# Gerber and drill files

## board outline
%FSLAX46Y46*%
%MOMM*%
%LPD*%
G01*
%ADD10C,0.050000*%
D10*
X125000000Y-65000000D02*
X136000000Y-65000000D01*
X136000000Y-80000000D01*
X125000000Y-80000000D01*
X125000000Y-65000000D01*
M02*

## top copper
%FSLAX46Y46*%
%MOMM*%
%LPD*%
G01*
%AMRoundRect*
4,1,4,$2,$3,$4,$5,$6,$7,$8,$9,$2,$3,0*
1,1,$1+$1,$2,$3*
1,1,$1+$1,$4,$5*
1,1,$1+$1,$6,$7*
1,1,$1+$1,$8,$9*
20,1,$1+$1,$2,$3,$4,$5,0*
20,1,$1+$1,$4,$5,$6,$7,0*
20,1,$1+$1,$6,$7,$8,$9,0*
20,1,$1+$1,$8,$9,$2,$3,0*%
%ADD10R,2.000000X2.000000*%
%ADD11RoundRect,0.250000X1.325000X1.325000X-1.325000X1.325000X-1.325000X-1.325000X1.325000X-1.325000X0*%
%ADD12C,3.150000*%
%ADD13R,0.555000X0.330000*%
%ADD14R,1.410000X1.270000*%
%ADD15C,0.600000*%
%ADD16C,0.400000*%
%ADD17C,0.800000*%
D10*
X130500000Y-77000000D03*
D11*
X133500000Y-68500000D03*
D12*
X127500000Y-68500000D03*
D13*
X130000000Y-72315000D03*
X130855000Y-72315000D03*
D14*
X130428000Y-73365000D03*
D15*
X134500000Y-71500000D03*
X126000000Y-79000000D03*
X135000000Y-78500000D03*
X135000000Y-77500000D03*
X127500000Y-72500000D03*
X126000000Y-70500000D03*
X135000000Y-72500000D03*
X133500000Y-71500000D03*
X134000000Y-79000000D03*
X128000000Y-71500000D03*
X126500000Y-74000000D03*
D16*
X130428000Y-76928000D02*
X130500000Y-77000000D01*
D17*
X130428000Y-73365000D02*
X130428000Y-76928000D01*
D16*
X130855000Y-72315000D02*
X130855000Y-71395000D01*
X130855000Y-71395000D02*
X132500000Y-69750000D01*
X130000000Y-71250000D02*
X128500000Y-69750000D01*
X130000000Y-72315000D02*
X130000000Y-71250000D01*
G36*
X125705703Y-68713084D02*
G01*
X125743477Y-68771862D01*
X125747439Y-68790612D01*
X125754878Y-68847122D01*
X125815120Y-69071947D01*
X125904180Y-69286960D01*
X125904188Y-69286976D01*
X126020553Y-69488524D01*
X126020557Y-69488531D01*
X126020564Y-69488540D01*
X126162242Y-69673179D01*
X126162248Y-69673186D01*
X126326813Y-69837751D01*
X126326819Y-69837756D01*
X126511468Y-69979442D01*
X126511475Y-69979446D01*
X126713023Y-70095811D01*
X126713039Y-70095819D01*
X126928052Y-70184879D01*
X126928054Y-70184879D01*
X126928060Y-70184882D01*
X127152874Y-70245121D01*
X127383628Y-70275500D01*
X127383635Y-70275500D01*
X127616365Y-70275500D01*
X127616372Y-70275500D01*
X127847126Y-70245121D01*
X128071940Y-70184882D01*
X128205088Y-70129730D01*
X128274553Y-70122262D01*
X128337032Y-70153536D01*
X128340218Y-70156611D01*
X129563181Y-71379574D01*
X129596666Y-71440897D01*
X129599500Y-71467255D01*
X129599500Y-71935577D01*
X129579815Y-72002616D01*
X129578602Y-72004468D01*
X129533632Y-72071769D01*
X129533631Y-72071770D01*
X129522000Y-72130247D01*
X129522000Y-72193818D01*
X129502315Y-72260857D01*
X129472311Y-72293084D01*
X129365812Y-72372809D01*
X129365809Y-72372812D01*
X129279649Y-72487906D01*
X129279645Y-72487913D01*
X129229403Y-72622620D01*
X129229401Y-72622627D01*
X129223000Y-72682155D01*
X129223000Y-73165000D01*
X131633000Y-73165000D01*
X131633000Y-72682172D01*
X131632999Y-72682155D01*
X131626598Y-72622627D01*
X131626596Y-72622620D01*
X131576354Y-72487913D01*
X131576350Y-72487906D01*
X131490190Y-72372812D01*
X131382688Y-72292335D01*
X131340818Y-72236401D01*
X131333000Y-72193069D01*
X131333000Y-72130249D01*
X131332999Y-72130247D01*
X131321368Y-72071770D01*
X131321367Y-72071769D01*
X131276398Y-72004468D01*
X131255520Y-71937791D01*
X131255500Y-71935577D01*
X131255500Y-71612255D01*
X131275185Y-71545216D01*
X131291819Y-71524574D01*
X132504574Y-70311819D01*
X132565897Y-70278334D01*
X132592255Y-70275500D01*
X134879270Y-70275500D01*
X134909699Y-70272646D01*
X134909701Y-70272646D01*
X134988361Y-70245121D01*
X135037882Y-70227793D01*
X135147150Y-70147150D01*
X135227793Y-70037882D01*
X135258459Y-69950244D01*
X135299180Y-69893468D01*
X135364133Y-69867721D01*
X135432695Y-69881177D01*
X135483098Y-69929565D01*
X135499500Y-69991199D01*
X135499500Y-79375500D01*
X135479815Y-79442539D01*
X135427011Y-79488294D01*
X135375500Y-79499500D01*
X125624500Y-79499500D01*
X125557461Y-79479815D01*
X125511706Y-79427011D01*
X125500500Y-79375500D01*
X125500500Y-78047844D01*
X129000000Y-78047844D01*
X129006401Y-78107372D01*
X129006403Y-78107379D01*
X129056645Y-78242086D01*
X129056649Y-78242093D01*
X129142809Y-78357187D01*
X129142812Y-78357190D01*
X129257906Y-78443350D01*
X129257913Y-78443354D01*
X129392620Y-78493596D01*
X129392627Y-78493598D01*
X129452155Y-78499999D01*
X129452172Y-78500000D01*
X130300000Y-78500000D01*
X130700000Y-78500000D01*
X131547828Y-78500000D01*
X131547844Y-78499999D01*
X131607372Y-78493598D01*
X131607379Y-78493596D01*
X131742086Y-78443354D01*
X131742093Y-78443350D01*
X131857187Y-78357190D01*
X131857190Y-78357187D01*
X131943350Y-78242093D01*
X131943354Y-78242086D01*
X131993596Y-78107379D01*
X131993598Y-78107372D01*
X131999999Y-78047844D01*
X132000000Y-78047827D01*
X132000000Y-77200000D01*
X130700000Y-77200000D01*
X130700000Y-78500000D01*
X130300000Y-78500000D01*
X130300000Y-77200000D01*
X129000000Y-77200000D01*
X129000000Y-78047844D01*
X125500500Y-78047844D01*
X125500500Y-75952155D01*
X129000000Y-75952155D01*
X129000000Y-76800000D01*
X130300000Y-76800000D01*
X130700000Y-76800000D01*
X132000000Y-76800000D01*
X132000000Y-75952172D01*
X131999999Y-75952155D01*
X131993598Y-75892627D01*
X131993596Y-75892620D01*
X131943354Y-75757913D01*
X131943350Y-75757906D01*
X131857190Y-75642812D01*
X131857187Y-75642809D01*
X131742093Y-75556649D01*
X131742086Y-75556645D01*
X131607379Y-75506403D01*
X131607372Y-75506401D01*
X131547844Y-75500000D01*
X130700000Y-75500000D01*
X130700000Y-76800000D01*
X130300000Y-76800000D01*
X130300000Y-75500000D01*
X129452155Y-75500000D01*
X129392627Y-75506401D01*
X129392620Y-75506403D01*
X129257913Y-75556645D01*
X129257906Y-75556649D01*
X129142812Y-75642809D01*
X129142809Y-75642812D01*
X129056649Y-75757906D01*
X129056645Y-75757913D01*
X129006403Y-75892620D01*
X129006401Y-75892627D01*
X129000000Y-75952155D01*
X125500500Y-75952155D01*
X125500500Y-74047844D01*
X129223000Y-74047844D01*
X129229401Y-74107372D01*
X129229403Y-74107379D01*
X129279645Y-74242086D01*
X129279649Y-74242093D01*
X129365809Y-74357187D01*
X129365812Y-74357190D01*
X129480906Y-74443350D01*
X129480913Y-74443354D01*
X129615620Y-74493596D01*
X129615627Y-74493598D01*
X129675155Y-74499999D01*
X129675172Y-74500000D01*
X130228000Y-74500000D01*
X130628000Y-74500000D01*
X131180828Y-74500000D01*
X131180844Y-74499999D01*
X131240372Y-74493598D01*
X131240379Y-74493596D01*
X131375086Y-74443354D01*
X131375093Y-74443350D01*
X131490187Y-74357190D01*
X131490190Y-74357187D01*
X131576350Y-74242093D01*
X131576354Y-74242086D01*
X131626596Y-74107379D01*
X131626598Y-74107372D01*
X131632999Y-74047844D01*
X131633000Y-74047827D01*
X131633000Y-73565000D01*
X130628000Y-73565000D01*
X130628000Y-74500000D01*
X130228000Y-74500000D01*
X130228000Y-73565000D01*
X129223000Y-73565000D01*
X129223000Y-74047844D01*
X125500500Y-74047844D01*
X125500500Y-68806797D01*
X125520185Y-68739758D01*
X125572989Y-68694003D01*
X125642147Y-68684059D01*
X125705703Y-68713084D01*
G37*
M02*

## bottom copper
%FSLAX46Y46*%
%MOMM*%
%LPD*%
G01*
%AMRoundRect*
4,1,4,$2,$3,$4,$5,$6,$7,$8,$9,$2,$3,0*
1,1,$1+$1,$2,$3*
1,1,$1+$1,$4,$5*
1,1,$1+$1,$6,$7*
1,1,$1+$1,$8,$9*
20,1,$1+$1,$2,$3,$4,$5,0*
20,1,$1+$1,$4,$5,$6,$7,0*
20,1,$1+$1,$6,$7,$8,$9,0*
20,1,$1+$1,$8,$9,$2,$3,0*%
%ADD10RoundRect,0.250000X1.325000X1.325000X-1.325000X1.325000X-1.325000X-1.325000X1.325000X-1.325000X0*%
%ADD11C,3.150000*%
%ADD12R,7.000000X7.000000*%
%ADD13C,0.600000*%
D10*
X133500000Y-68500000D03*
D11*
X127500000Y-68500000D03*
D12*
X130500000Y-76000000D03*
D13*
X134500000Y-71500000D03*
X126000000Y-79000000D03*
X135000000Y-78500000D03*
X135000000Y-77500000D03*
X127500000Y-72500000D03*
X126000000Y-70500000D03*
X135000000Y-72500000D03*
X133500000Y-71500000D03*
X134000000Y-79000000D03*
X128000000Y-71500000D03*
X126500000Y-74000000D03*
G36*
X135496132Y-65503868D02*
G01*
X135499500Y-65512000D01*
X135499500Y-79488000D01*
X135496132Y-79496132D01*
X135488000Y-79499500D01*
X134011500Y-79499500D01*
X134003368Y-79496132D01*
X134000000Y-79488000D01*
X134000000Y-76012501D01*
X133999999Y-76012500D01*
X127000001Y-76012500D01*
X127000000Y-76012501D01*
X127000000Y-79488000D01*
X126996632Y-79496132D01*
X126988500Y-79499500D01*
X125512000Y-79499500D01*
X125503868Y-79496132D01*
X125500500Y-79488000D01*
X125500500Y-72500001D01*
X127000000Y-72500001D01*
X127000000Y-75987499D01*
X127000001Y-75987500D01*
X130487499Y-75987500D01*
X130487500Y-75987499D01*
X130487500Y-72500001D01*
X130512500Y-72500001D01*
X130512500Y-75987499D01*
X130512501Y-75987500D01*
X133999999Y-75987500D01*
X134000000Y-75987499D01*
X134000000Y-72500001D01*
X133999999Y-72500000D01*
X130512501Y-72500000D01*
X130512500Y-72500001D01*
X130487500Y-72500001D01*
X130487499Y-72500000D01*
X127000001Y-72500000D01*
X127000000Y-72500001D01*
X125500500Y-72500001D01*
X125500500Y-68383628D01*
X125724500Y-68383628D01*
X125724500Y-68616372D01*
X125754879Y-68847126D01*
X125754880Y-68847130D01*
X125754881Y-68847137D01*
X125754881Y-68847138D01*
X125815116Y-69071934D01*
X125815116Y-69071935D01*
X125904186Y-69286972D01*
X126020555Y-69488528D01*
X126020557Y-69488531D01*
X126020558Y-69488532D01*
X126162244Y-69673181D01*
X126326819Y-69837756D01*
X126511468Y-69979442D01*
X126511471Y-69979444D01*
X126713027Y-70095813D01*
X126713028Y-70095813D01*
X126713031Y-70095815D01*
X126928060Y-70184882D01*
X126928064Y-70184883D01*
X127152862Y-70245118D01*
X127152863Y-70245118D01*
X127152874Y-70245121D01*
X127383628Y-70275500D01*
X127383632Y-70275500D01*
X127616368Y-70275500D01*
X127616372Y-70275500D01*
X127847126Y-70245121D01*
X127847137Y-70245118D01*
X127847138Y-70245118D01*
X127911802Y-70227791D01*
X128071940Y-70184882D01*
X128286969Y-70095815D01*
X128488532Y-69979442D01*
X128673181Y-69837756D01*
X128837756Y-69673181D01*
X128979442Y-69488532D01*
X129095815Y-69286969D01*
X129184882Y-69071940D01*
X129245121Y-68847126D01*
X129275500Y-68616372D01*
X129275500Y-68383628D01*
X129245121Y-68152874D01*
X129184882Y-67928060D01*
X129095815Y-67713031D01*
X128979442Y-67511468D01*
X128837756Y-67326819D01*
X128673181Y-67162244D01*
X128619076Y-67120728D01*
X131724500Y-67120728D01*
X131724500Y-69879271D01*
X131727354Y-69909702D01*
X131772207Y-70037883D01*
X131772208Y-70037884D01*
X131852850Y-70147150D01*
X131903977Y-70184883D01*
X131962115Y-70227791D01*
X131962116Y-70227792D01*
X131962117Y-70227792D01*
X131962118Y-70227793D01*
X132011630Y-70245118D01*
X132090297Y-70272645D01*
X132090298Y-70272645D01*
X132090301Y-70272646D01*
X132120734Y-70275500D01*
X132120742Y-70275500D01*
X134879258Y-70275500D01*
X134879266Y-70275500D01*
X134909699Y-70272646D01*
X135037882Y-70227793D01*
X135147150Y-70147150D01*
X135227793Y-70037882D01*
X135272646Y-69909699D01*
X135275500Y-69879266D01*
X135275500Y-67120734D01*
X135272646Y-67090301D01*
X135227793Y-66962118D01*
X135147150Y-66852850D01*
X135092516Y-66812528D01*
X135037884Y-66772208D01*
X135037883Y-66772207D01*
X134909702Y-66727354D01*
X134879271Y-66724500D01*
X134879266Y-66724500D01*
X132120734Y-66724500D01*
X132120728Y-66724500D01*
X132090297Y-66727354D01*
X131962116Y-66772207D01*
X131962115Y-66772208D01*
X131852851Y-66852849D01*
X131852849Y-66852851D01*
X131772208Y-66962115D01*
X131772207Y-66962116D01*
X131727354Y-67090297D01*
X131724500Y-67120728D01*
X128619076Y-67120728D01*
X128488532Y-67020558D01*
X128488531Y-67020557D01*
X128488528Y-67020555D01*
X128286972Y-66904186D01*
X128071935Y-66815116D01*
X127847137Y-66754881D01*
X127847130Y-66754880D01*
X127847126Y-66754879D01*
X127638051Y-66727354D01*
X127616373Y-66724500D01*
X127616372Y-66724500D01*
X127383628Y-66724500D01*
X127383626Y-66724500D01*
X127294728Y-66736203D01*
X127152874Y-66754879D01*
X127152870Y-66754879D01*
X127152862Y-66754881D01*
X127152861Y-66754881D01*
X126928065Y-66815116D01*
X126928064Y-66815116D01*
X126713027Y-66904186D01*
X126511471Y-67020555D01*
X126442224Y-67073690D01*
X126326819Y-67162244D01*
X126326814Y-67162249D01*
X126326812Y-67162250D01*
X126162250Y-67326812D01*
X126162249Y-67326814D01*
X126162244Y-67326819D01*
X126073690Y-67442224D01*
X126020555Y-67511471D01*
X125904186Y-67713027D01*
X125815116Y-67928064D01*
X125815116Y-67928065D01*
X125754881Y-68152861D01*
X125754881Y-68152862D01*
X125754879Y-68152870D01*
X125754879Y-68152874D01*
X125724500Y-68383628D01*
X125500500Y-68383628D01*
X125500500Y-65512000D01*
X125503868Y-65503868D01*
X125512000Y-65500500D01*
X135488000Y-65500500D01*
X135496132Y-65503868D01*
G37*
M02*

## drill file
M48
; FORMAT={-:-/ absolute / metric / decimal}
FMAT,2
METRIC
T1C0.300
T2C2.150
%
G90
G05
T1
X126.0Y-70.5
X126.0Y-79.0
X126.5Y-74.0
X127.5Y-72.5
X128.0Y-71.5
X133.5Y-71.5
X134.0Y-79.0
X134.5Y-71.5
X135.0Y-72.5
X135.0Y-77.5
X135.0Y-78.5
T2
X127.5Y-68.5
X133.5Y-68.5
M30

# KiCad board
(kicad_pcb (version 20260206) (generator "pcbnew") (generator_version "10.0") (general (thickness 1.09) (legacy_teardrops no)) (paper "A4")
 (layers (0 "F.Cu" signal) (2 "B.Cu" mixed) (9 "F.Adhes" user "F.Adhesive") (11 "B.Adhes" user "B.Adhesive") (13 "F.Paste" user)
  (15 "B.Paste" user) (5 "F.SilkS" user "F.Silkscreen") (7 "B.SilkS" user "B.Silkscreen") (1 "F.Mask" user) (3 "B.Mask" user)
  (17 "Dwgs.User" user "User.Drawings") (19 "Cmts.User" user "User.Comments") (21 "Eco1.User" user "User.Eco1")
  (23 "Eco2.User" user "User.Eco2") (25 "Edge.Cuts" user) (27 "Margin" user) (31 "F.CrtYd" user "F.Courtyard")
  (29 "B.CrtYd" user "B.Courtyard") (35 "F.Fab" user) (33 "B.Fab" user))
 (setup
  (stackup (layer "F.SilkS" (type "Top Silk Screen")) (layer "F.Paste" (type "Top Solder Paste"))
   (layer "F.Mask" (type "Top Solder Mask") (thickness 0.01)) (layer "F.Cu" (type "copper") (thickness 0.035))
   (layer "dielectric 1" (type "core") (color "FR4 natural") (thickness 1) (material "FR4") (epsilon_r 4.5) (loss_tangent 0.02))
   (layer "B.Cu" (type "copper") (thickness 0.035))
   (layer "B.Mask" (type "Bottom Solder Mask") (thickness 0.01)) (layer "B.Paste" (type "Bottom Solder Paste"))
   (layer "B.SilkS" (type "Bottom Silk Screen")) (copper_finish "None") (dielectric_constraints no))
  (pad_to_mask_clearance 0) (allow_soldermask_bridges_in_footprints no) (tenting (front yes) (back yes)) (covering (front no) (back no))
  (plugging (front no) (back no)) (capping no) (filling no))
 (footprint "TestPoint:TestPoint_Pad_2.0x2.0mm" (layer "F.Cu") (at 130.5 77)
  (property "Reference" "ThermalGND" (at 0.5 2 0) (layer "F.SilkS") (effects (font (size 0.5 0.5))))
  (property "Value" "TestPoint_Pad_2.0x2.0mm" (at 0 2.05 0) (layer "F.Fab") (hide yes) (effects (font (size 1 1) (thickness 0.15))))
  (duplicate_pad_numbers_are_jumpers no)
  (pad "1" smd rect (at 0 0) (size 2 2) (layers "F.Cu" "F.Mask") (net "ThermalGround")))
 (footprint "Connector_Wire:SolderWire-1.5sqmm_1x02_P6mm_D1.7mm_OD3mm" (layer "F.Cu") (at 133.5 68.5 180)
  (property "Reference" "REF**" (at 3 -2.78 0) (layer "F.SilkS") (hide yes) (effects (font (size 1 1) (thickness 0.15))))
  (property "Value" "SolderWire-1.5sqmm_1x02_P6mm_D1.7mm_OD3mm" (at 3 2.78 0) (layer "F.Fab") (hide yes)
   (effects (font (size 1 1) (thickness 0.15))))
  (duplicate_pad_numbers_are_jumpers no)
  (pad "1" thru_hole roundrect (at 0 0 180) (size 3.15 3.15) (drill 2.15) (layers "*.Cu" "*.Mask") (remove_unused_layers no)
   (roundrect_rratio 0.079365) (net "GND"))
  (pad "2" thru_hole circle (at 6 0 180) (size 3.15 3.15) (drill 2.15) (layers "*.Cu" "*.Mask") (remove_unused_layers no) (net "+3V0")))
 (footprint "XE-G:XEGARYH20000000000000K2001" (layer "F.Cu") (at 130.428 73.075)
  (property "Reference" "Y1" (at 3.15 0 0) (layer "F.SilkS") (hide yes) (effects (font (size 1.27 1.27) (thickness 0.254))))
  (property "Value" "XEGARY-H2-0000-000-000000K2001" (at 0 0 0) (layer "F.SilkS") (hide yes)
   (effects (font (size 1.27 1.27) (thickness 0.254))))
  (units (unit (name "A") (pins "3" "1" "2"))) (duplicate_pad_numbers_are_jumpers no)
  (pad "1" smd rect (at -0.428 -0.76 90) (size 0.33 0.555) (layers "F.Cu" "F.Mask" "F.Paste") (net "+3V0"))
  (pad "2" smd rect (at 0.427 -0.76 90) (size 0.33 0.555) (layers "F.Cu" "F.Mask" "F.Paste") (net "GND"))
  (pad "3" smd rect (at 0 0.29 90) (size 1.27 1.41) (layers "F.Cu" "F.Mask" "F.Paste") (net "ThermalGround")))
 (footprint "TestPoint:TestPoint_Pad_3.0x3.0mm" (layer "B.Cu") (at 130.5 76 180)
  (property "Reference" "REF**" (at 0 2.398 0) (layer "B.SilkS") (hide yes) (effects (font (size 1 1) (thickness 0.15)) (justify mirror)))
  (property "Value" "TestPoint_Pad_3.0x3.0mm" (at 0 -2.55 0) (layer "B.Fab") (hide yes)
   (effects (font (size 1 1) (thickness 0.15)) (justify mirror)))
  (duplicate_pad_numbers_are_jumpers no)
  (pad "1" smd rect (at 0 0 180) (size 7 7) (layers "B.Cu" "B.Mask") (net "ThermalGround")))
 (gr_rect (start 125 65) (end 136 80) (stroke (width 0.05) (type default)) (fill no) (layer "Edge.Cuts"))
 (segment (start 130.428 76.928) (end 130.5 77) (width 0.4) (layer "F.Cu") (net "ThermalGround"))
 (segment (start 130.428 73.365) (end 130.428 76.928) (width 0.8) (layer "F.Cu") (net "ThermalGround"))
 (via (at 134.5 71.5) (size 0.6) (drill 0.3) (layers "F.Cu" "B.Cu") (free yes) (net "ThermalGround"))
 (via (at 126 79) (size 0.6) (drill 0.3) (layers "F.Cu" "B.Cu") (free yes) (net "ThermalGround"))
 (via (at 135 78.5) (size 0.6) (drill 0.3) (layers "F.Cu" "B.Cu") (free yes) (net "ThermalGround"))
 (via (at 135 77.5) (size 0.6) (drill 0.3) (layers "F.Cu" "B.Cu") (free yes) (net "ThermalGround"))
 (via (at 127.5 72.5) (size 0.6) (drill 0.3) (layers "F.Cu" "B.Cu") (free yes) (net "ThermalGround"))
 (via (at 126 70.5) (size 0.6) (drill 0.3) (layers "F.Cu" "B.Cu") (free yes) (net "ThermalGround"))
 (via (at 135 72.5) (size 0.6) (drill 0.3) (layers "F.Cu" "B.Cu") (free yes) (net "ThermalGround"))
 (via (at 133.5 71.5) (size 0.6) (drill 0.3) (layers "F.Cu" "B.Cu") (free yes) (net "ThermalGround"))
 (via (at 134 79) (size 0.6) (drill 0.3) (layers "F.Cu" "B.Cu") (free yes) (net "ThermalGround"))
 (via (at 128 71.5) (size 0.6) (drill 0.3) (layers "F.Cu" "B.Cu") (free yes) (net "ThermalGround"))
 (via (at 126.5 74) (size 0.6) (drill 0.3) (layers "F.Cu" "B.Cu") (free yes) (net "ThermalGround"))
 (segment (start 130.855 72.315) (end 130.855 71.395) (width 0.4) (layer "F.Cu") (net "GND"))
 (segment (start 130.855 71.395) (end 132.5 69.75) (width 0.4) (layer "F.Cu") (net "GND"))
 (segment (start 130 71.25) (end 128.5 69.75) (width 0.4) (layer "F.Cu") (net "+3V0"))
 (segment (start 130 72.315) (end 130 71.25) (width 0.4) (layer "F.Cu") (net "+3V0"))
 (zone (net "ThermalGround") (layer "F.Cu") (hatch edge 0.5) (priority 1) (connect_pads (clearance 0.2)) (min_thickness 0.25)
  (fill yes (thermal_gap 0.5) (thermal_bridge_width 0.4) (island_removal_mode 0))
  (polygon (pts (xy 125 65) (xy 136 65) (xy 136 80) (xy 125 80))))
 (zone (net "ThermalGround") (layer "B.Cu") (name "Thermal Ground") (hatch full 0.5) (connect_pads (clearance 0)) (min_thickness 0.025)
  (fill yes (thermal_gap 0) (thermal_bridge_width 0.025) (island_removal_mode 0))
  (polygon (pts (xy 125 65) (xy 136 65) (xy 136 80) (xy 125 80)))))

